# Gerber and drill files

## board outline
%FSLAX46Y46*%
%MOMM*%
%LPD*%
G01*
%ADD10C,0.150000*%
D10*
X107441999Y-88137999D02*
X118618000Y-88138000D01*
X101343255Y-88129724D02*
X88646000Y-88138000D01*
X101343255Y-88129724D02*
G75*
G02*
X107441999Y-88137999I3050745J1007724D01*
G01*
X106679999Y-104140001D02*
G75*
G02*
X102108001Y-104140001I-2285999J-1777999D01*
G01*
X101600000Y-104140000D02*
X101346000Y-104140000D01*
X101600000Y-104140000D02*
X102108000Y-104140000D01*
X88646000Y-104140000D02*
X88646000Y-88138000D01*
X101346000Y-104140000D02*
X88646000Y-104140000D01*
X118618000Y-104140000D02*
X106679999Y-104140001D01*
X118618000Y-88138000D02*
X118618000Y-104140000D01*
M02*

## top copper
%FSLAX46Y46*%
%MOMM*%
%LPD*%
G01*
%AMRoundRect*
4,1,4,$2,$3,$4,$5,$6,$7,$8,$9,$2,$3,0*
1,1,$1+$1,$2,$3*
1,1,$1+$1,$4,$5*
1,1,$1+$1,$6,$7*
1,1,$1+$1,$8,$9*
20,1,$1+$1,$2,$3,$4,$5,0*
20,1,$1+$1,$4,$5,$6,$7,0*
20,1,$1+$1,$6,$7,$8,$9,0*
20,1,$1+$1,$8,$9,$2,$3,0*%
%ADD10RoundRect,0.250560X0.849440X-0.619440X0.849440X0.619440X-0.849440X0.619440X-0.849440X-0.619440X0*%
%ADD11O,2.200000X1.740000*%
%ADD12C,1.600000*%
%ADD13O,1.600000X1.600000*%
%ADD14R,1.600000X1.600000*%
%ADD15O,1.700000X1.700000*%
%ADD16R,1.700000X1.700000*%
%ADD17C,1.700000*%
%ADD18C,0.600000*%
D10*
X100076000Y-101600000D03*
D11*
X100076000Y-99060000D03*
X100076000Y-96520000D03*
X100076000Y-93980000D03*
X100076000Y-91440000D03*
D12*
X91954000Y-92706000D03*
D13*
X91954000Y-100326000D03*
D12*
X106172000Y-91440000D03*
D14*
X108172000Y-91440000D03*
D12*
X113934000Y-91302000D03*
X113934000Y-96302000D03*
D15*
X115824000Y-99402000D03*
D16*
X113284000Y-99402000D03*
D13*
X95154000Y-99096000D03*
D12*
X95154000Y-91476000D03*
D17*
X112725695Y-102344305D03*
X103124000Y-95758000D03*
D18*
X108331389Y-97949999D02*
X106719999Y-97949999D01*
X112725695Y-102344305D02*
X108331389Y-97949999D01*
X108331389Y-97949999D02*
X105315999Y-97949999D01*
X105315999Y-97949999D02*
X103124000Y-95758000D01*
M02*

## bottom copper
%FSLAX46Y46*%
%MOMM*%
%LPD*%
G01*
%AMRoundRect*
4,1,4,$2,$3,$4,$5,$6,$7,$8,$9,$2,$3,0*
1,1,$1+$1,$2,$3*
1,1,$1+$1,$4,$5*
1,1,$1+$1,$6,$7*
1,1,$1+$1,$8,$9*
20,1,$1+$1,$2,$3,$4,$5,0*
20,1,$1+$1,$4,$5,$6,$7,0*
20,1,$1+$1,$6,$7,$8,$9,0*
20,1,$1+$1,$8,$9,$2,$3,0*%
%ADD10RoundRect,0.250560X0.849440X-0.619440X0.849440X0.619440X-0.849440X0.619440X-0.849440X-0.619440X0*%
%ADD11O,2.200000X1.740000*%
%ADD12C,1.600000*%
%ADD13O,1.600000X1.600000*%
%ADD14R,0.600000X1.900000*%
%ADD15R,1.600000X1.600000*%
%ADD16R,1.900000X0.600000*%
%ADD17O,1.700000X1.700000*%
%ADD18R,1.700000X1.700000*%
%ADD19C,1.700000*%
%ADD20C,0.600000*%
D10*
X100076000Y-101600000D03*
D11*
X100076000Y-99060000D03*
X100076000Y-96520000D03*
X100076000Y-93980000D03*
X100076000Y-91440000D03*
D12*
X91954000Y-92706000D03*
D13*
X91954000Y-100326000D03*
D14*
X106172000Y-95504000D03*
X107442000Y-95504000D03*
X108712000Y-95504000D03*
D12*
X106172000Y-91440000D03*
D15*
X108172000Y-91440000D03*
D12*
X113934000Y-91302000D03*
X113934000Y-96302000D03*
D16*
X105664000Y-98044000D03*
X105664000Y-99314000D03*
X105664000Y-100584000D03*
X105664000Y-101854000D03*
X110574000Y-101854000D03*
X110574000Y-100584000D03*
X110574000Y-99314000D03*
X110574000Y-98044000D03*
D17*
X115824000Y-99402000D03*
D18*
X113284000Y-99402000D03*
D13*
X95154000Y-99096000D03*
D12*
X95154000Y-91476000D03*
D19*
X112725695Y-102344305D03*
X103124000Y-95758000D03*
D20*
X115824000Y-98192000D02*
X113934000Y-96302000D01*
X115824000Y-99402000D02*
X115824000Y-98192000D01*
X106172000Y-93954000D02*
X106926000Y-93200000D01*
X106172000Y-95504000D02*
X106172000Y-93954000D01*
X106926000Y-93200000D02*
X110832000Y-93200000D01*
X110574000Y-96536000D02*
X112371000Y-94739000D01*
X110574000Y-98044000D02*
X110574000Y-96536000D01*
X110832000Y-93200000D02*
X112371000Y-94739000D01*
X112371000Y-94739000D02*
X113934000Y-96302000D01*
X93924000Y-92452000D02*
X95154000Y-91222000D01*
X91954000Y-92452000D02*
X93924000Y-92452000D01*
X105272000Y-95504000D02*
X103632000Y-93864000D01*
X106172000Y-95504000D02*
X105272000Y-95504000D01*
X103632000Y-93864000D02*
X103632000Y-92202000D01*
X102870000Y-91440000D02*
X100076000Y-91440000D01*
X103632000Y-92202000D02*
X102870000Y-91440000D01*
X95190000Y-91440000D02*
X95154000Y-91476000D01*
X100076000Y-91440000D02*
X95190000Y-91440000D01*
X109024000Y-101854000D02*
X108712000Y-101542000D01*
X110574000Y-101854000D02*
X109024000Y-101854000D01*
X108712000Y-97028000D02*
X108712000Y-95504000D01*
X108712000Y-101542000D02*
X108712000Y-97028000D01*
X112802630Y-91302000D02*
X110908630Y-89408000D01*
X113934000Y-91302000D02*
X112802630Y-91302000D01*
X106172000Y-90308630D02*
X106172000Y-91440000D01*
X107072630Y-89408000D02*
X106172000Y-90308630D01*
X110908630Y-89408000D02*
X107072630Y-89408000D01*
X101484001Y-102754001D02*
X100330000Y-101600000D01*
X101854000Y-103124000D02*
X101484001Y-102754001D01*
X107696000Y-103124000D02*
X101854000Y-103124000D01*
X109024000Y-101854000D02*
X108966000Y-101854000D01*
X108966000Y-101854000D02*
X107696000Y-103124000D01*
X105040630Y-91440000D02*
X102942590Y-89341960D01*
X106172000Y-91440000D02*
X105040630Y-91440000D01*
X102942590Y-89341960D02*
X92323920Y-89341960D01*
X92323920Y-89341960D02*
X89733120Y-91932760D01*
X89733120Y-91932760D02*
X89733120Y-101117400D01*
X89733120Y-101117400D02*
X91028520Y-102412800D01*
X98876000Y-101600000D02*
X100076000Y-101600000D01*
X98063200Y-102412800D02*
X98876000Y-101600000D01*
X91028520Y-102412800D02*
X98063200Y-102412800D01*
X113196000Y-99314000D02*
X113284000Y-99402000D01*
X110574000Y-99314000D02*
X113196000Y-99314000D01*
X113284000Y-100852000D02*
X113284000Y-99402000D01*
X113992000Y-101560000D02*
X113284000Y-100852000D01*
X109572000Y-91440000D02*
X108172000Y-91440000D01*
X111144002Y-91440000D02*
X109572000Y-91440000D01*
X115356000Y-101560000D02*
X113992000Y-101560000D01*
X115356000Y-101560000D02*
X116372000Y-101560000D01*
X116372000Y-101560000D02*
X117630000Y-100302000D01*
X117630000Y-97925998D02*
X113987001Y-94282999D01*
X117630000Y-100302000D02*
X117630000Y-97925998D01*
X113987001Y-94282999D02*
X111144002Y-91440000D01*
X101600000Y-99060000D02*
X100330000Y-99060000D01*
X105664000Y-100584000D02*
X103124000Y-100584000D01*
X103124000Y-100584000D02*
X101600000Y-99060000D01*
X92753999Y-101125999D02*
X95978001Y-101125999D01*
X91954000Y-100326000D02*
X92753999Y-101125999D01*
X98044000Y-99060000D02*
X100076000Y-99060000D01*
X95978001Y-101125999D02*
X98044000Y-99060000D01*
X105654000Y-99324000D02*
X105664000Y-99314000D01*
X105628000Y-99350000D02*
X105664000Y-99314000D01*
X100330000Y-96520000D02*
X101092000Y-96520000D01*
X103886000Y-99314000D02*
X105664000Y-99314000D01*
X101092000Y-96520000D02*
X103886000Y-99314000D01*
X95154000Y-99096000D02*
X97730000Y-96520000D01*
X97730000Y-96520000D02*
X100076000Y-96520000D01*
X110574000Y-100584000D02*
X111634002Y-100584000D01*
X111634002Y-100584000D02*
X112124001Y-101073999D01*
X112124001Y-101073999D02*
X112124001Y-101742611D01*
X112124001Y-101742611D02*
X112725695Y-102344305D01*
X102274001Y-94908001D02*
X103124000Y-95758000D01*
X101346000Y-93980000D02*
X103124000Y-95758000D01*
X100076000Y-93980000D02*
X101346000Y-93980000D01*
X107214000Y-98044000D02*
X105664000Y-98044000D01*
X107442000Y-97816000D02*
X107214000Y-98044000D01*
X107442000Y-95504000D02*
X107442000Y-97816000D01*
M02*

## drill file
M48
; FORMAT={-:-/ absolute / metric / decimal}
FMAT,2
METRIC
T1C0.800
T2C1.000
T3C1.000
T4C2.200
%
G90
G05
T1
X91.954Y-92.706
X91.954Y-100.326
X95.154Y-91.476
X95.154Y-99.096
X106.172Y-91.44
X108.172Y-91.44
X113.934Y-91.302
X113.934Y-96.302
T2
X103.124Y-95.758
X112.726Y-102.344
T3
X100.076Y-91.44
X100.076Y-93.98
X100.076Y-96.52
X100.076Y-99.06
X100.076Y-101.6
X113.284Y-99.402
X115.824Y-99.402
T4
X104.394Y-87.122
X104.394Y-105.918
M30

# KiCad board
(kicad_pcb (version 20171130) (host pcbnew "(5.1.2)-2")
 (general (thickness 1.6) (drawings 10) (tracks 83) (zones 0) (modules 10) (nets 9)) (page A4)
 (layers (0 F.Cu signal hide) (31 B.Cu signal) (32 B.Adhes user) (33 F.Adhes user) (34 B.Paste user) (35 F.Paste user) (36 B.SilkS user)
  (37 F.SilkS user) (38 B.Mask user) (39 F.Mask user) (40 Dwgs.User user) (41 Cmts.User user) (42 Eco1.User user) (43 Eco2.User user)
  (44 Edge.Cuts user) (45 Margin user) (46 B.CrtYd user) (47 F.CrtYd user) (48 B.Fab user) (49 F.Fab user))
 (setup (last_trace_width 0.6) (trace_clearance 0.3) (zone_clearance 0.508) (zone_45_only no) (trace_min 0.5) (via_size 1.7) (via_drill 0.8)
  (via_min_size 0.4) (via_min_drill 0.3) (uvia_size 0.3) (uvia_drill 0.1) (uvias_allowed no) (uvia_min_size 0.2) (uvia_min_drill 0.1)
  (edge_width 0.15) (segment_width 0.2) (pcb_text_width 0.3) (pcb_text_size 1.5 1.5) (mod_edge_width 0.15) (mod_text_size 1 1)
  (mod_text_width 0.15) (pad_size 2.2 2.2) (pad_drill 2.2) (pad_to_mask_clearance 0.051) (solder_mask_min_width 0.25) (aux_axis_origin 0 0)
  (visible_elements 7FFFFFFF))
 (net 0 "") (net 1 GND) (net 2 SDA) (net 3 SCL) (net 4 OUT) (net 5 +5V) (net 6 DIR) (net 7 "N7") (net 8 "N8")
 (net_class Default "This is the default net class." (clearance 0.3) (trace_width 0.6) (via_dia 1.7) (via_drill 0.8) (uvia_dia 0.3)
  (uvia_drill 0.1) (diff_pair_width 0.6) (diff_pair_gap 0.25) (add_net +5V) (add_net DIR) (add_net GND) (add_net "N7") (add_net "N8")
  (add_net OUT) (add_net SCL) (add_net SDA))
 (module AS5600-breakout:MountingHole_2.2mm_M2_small (layer F.Cu) (at 104.394 105.918)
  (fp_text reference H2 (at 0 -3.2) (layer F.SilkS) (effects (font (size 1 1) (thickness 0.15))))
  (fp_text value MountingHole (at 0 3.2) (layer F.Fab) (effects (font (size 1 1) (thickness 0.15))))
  (pad 1 np_thru_hole circle (at 0 0) (size 2.2 2.2) (drill 2.2) (layers *.Cu *.Mask)))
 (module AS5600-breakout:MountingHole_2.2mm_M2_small (layer F.Cu) (at 104.394 87.122)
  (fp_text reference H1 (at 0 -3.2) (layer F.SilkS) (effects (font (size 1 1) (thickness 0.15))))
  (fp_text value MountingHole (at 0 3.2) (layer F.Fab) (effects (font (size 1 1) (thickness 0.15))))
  (pad "" np_thru_hole circle (at 0 0) (size 2.2 2.2) (drill 2.2) (layers *.Cu *.Mask)))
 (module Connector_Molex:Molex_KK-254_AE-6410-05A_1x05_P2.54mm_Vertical (layer F.Cu) (at 100.076 101.6 90)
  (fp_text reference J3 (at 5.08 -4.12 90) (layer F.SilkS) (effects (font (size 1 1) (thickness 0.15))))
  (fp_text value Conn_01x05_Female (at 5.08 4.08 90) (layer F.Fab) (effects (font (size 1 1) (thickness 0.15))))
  (pad 1 thru_hole roundrect (at 0 0 90) (size 1.74 2.2) (drill 1) (layers *.Cu *.Mask) (roundrect_rratio 0.144) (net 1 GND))
  (pad 2 thru_hole oval (at 2.54 0 90) (size 1.74 2.2) (drill 1) (layers *.Cu *.Mask) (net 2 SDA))
  (pad 3 thru_hole oval (at 5.08 0 90) (size 1.74 2.2) (drill 1) (layers *.Cu *.Mask) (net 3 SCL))
  (pad 4 thru_hole oval (at 7.62 0 90) (size 1.74 2.2) (drill 1) (layers *.Cu *.Mask) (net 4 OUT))
  (pad 5 thru_hole oval (at 10.16 0 90) (size 1.74 2.2) (drill 1) (layers *.Cu *.Mask) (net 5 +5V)))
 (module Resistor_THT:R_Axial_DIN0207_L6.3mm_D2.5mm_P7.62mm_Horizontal (layer F.Cu) (at 91.954 92.706 270)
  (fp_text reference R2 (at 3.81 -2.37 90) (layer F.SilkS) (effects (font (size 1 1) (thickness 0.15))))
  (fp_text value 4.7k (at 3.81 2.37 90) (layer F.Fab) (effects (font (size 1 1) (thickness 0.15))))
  (pad 1 thru_hole circle (at 0 0 270) (size 1.6 1.6) (drill 0.8) (layers *.Cu *.Mask) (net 5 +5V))
  (pad 2 thru_hole oval (at 7.62 0 270) (size 1.6 1.6) (drill 0.8) (layers *.Cu *.Mask) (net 2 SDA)))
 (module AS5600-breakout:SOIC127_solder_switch (layer B.Cu) (at 106.807 93.049 90)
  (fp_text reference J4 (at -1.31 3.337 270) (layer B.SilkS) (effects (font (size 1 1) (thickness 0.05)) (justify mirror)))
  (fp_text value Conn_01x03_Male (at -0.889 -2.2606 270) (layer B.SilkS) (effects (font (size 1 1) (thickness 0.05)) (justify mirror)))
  (pad 3 smd rect (at -2.455 -0.635 90) (size 1.9 0.6) (layers B.Cu B.Paste B.Mask) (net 5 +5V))
  (pad 2 smd rect (at -2.455 0.635 90) (size 1.9 0.6) (layers B.Cu B.Paste B.Mask) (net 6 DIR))
  (pad 1 smd rect (at -2.455 1.905 90) (size 1.9 0.6) (layers B.Cu B.Paste B.Mask) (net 1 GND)))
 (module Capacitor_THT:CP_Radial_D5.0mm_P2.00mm (layer F.Cu) (at 108.172 91.44 180)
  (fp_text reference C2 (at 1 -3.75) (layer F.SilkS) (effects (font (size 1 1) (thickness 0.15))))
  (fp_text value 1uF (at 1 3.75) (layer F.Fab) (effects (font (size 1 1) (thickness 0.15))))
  (pad 2 thru_hole circle (at 2 0 180) (size 1.6 1.6) (drill 0.8) (layers *.Cu *.Mask) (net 1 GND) (clearance 0.2))
  (pad 1 thru_hole rect (at 0 0 180) (size 1.6 1.6) (drill 0.8) (layers *.Cu *.Mask) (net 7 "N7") (clearance 0.2)))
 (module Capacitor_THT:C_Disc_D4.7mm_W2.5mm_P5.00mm (layer F.Cu) (at 113.934 96.302 90)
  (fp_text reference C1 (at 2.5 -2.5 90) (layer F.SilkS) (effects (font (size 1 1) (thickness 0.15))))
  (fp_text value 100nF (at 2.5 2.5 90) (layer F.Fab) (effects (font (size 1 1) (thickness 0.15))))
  (pad 2 thru_hole circle (at 5 0 90) (size 1.6 1.6) (drill 0.8) (layers *.Cu *.Mask) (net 1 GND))
  (pad 1 thru_hole circle (at 0 0 90) (size 1.6 1.6) (drill 0.8) (layers *.Cu *.Mask) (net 5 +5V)))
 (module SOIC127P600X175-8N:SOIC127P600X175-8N (layer B.Cu) (at 108.119 99.949 180)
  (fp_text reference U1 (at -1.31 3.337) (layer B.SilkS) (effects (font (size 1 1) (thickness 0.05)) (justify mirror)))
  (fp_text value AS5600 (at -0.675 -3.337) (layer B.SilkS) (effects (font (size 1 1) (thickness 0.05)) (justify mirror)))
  (pad 8 smd rect (at 2.455 1.905 180) (size 1.9 0.6) (layers B.Cu B.Paste B.Mask) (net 6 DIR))
  (pad 7 smd rect (at 2.455 0.635 180) (size 1.9 0.6) (layers B.Cu B.Paste B.Mask) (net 3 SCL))
  (pad 6 smd rect (at 2.455 -0.635 180) (size 1.9 0.6) (layers B.Cu B.Paste B.Mask) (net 2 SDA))
  (pad 5 smd rect (at 2.455 -1.905 180) (size 1.9 0.6) (layers B.Cu B.Paste B.Mask) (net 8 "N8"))
  (pad 4 smd rect (at -2.455 -1.905 180) (size 1.9 0.6) (layers B.Cu B.Paste B.Mask) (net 1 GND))
  (pad 3 smd rect (at -2.455 -0.635 180) (size 1.9 0.6) (layers B.Cu B.Paste B.Mask) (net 4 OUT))
  (pad 2 smd rect (at -2.455 0.635 180) (size 1.9 0.6) (layers B.Cu B.Paste B.Mask) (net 7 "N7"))
  (pad 1 smd rect (at -2.455 1.905 180) (size 1.9 0.6) (layers B.Cu B.Paste B.Mask) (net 5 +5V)))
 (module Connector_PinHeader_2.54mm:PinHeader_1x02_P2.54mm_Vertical (layer F.Cu) (at 113.284 99.402 90)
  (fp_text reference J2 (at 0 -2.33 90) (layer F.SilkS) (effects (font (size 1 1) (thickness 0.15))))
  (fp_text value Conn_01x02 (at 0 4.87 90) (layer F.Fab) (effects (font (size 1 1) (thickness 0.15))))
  (pad 2 thru_hole oval (at 0 2.54 90) (size 1.7 1.7) (drill 1) (layers *.Cu *.Mask) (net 5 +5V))
  (pad 1 thru_hole rect (at 0 0 90) (size 1.7 1.7) (drill 1) (layers *.Cu *.Mask) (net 7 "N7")))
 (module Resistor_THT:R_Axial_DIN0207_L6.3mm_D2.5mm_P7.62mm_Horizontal (layer F.Cu) (at 95.154 91.476 270)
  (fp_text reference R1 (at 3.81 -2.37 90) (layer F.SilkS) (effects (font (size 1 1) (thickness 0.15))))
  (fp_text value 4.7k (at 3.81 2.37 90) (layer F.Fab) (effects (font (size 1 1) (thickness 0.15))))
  (pad 2 thru_hole oval (at 7.62 0 270) (size 1.6 1.6) (drill 0.8) (layers *.Cu *.Mask) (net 3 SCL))
  (pad 1 thru_hole circle (at 0 0 270) (size 1.6 1.6) (drill 0.8) (layers *.Cu *.Mask) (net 5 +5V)))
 (gr_line (start 107.441999 88.137999) (end 118.618 88.138) (layer Edge.Cuts) (width 0.15))
 (gr_line (start 101.343255 88.129724) (end 88.646 88.138) (layer Edge.Cuts) (width 0.15))
 (gr_arc (start 104.394 87.122) (end 107.441999 88.137999) (angle -216.714395) (layer Edge.Cuts) (width 0.15))
 (gr_arc (start 104.394 105.918) (end 102.108001 104.140001) (angle -255.7499673) (layer Edge.Cuts) (width 0.15))
 (gr_line (start 101.6 104.14) (end 101.346 104.14) (layer Edge.Cuts) (width 0.15))
 (gr_line (start 101.6 104.14) (end 102.108 104.14) (layer Edge.Cuts) (width 0.15))
 (gr_line (start 88.646 104.14) (end 88.646 88.138) (layer Edge.Cuts) (width 0.15))
 (gr_line (start 101.346 104.14) (end 88.646 104.14) (layer Edge.Cuts) (width 0.15))
 (gr_line (start 118.618 104.14) (end 106.679999 104.140001) (layer Edge.Cuts) (width 0.15))
 (gr_line (start 118.618 88.138) (end 118.618 104.14) (layer Edge.Cuts) (width 0.15))
 (segment (start 115.824 98.192) (end 113.934 96.302) (width 0.6) (layer B.Cu) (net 5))
 (segment (start 115.824 99.402) (end 115.824 98.192) (width 0.6) (layer B.Cu) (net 5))
 (segment (start 106.172 93.954) (end 106.926 93.2) (width 0.6) (layer B.Cu) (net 5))
 (segment (start 106.172 95.504) (end 106.172 93.954) (width 0.6) (layer B.Cu) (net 5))
 (segment (start 106.926 93.2) (end 110.832 93.2) (width 0.6) (layer B.Cu) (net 5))
 (segment (start 110.574 96.536) (end 112.371 94.739) (width 0.6) (layer B.Cu) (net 5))
 (segment (start 110.574 98.044) (end 110.574 96.536) (width 0.6) (layer B.Cu) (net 5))
 (segment (start 110.832 93.2) (end 112.371 94.739) (width 0.6) (layer B.Cu) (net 5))
 (segment (start 112.371 94.739) (end 113.934 96.302) (width 0.6) (layer B.Cu) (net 5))
 (segment (start 93.924 92.452) (end 95.154 91.222) (width 0.6) (layer B.Cu) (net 5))
 (segment (start 91.954 92.452) (end 93.924 92.452) (width 0.6) (layer B.Cu) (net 5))
 (segment (start 105.272 95.504) (end 103.632 93.864) (width 0.6) (layer B.Cu) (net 5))
 (segment (start 106.172 95.504) (end 105.272 95.504) (width 0.6) (layer B.Cu) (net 5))
 (segment (start 103.632 93.864) (end 103.632 92.202) (width 0.6) (layer B.Cu) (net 5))
 (segment (start 102.87 91.44) (end 100.076 91.44) (width 0.6) (layer B.Cu) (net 5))
 (segment (start 103.632 92.202) (end 102.87 91.44) (width 0.6) (layer B.Cu) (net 5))
 (segment (start 95.19 91.44) (end 95.154 91.476) (width 0.6) (layer B.Cu) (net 5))
 (segment (start 100.076 91.44) (end 95.19 91.44) (width 0.6) (layer B.Cu) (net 5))
 (segment (start 109.024 101.854) (end 108.712 101.542) (width 0.6) (layer B.Cu) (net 1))
 (segment (start 110.574 101.854) (end 109.024 101.854) (width 0.6) (layer B.Cu) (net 1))
 (segment (start 108.712 97.028) (end 108.712 95.504) (width 0.6) (layer B.Cu) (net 1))
 (segment (start 108.712 101.542) (end 108.712 97.028) (width 0.6) (layer B.Cu) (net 1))
 (segment (start 112.80263 91.302) (end 110.90863 89.408) (width 0.6) (layer B.Cu) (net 1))
 (segment (start 113.934 91.302) (end 112.80263 91.302) (width 0.6) (layer B.Cu) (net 1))
 (segment (start 106.172 90.30863) (end 106.172 91.44) (width 0.6) (layer B.Cu) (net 1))
 (segment (start 107.07263 89.408) (end 106.172 90.30863) (width 0.6) (layer B.Cu) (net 1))
 (segment (start 110.90863 89.408) (end 107.07263 89.408) (width 0.6) (layer B.Cu) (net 1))
 (segment (start 101.484001 102.754001) (end 100.33 101.6) (width 0.6) (layer B.Cu) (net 1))
 (segment (start 101.854 103.124) (end 101.484001 102.754001) (width 0.6) (layer B.Cu) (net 1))
 (segment (start 107.696 103.124) (end 101.854 103.124) (width 0.6) (layer B.Cu) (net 1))
 (segment (start 109.024 101.854) (end 108.966 101.854) (width 0.6) (layer B.Cu) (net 1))
 (segment (start 108.966 101.854) (end 107.696 103.124) (width 0.6) (layer B.Cu) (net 1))
 (segment (start 105.04063 91.44) (end 102.94259 89.34196) (width 0.6) (layer B.Cu) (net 1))
 (segment (start 106.172 91.44) (end 105.04063 91.44) (width 0.6) (layer B.Cu) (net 1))
 (segment (start 102.94259 89.34196) (end 92.32392 89.34196) (width 0.6) (layer B.Cu) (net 1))
 (segment (start 92.32392 89.34196) (end 89.73312 91.93276) (width 0.6) (layer B.Cu) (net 1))
 (segment (start 89.73312 91.93276) (end 89.73312 101.1174) (width 0.6) (layer B.Cu) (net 1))
 (segment (start 89.73312 101.1174) (end 91.02852 102.4128) (width 0.6) (layer B.Cu) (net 1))
 (segment (start 98.876 101.6) (end 100.076 101.6) (width 0.6) (layer B.Cu) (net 1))
 (segment (start 98.0632 102.4128) (end 98.876 101.6) (width 0.6) (layer B.Cu) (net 1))
 (segment (start 91.02852 102.4128) (end 98.0632 102.4128) (width 0.6) (layer B.Cu) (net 1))
 (segment (start 113.196 99.314) (end 113.284 99.402) (width 0.6) (layer B.Cu) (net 7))
 (segment (start 110.574 99.314) (end 113.196 99.314) (width 0.6) (layer B.Cu) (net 7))
 (segment (start 113.284 100.852) (end 113.284 99.402) (width 0.6) (layer B.Cu) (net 7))
 (segment (start 113.992 101.56) (end 113.284 100.852) (width 0.6) (layer B.Cu) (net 7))
 (segment (start 109.572 91.44) (end 108.172 91.44) (width 0.6) (layer B.Cu) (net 7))
 (segment (start 111.144002 91.44) (end 109.572 91.44) (width 0.6) (layer B.Cu) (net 7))
 (segment (start 115.356 101.56) (end 113.992 101.56) (width 0.6) (layer B.Cu) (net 7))
 (segment (start 115.356 101.56) (end 116.372 101.56) (width 0.6) (layer B.Cu) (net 7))
 (segment (start 116.372 101.56) (end 117.63 100.302) (width 0.6) (layer B.Cu) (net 7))
 (segment (start 117.63 97.925998) (end 113.987001 94.282999) (width 0.6) (layer B.Cu) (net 7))
 (segment (start 117.63 100.302) (end 117.63 97.925998) (width 0.6) (layer B.Cu) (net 7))
 (segment (start 113.987001 94.282999) (end 111.144002 91.44) (width 0.6) (layer B.Cu) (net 7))
 (segment (start 101.6 99.06) (end 100.33 99.06) (width 0.6) (layer B.Cu) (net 2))
 (segment (start 105.664 100.584) (end 103.124 100.584) (width 0.6) (layer B.Cu) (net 2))
 (segment (start 103.124 100.584) (end 101.6 99.06) (width 0.6) (layer B.Cu) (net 2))
 (segment (start 92.753999 101.125999) (end 95.978001 101.125999) (width 0.6) (layer B.Cu) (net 2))
 (segment (start 91.954 100.326) (end 92.753999 101.125999) (width 0.6) (layer B.Cu) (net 2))
 (segment (start 98.044 99.06) (end 100.076 99.06) (width 0.6) (layer B.Cu) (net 2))
 (segment (start 95.978001 101.125999) (end 98.044 99.06) (width 0.6) (layer B.Cu) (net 2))
 (segment (start 105.654 99.324) (end 105.664 99.314) (width 0.6) (layer B.Cu) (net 3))
 (segment (start 105.628 99.35) (end 105.664 99.314) (width 0.6) (layer B.Cu) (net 3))
 (segment (start 100.33 96.52) (end 101.092 96.52) (width 0.6) (layer B.Cu) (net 3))
 (segment (start 103.886 99.314) (end 105.664 99.314) (width 0.6) (layer B.Cu) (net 3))
 (segment (start 101.092 96.52) (end 103.886 99.314) (width 0.6) (layer B.Cu) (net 3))
 (segment (start 95.154 99.096) (end 97.73 96.52) (width 0.6) (layer B.Cu) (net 3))
 (segment (start 97.73 96.52) (end 100.076 96.52) (width 0.6) (layer B.Cu) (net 3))
 (segment (start 110.574 100.584) (end 111.634002 100.584) (width 0.6) (layer B.Cu) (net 4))
 (segment (start 111.634002 100.584) (end 112.124001 101.073999) (width 0.6) (layer B.Cu) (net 4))
 (via (at 112.725695 102.344305) (size 1.7) (drill 1) (layers F.Cu B.Cu) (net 4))
 (segment (start 112.124001 101.073999) (end 112.124001 101.742611) (width 0.6) (layer B.Cu) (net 4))
 (segment (start 112.124001 101.742611) (end 112.725695 102.344305) (width 0.6) (layer B.Cu) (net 4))
 (segment (start 108.331389 97.949999) (end 106.719999 97.949999) (width 0.6) (layer F.Cu) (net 4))
 (segment (start 112.725695 102.344305) (end 108.331389 97.949999) (width 0.6) (layer F.Cu) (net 4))
 (via (at 103.124 95.758) (size 1.7) (drill 1) (layers F.Cu B.Cu) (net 4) (status 1000000))
 (segment (start 108.331389 97.949999) (end 105.315999 97.949999) (width 0.6) (layer F.Cu) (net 4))
 (segment (start 105.315999 97.949999) (end 103.124 95.758) (width 0.6) (layer F.Cu) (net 4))
 (segment (start 102.274001 94.908001) (end 103.124 95.758) (width 0.6) (layer B.Cu) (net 4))
 (segment (start 101.346 93.98) (end 103.124 95.758) (width 0.6) (layer B.Cu) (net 4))
 (segment (start 100.076 93.98) (end 101.346 93.98) (width 0.6) (layer B.Cu) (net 4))
 (segment (start 107.214 98.044) (end 105.664 98.044) (width 0.6) (layer B.Cu) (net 6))
 (segment (start 107.442 97.816) (end 107.214 98.044) (width 0.6) (layer B.Cu) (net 6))
 (segment (start 107.442 95.504) (end 107.442 97.816) (width 0.6) (layer B.Cu) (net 6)))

